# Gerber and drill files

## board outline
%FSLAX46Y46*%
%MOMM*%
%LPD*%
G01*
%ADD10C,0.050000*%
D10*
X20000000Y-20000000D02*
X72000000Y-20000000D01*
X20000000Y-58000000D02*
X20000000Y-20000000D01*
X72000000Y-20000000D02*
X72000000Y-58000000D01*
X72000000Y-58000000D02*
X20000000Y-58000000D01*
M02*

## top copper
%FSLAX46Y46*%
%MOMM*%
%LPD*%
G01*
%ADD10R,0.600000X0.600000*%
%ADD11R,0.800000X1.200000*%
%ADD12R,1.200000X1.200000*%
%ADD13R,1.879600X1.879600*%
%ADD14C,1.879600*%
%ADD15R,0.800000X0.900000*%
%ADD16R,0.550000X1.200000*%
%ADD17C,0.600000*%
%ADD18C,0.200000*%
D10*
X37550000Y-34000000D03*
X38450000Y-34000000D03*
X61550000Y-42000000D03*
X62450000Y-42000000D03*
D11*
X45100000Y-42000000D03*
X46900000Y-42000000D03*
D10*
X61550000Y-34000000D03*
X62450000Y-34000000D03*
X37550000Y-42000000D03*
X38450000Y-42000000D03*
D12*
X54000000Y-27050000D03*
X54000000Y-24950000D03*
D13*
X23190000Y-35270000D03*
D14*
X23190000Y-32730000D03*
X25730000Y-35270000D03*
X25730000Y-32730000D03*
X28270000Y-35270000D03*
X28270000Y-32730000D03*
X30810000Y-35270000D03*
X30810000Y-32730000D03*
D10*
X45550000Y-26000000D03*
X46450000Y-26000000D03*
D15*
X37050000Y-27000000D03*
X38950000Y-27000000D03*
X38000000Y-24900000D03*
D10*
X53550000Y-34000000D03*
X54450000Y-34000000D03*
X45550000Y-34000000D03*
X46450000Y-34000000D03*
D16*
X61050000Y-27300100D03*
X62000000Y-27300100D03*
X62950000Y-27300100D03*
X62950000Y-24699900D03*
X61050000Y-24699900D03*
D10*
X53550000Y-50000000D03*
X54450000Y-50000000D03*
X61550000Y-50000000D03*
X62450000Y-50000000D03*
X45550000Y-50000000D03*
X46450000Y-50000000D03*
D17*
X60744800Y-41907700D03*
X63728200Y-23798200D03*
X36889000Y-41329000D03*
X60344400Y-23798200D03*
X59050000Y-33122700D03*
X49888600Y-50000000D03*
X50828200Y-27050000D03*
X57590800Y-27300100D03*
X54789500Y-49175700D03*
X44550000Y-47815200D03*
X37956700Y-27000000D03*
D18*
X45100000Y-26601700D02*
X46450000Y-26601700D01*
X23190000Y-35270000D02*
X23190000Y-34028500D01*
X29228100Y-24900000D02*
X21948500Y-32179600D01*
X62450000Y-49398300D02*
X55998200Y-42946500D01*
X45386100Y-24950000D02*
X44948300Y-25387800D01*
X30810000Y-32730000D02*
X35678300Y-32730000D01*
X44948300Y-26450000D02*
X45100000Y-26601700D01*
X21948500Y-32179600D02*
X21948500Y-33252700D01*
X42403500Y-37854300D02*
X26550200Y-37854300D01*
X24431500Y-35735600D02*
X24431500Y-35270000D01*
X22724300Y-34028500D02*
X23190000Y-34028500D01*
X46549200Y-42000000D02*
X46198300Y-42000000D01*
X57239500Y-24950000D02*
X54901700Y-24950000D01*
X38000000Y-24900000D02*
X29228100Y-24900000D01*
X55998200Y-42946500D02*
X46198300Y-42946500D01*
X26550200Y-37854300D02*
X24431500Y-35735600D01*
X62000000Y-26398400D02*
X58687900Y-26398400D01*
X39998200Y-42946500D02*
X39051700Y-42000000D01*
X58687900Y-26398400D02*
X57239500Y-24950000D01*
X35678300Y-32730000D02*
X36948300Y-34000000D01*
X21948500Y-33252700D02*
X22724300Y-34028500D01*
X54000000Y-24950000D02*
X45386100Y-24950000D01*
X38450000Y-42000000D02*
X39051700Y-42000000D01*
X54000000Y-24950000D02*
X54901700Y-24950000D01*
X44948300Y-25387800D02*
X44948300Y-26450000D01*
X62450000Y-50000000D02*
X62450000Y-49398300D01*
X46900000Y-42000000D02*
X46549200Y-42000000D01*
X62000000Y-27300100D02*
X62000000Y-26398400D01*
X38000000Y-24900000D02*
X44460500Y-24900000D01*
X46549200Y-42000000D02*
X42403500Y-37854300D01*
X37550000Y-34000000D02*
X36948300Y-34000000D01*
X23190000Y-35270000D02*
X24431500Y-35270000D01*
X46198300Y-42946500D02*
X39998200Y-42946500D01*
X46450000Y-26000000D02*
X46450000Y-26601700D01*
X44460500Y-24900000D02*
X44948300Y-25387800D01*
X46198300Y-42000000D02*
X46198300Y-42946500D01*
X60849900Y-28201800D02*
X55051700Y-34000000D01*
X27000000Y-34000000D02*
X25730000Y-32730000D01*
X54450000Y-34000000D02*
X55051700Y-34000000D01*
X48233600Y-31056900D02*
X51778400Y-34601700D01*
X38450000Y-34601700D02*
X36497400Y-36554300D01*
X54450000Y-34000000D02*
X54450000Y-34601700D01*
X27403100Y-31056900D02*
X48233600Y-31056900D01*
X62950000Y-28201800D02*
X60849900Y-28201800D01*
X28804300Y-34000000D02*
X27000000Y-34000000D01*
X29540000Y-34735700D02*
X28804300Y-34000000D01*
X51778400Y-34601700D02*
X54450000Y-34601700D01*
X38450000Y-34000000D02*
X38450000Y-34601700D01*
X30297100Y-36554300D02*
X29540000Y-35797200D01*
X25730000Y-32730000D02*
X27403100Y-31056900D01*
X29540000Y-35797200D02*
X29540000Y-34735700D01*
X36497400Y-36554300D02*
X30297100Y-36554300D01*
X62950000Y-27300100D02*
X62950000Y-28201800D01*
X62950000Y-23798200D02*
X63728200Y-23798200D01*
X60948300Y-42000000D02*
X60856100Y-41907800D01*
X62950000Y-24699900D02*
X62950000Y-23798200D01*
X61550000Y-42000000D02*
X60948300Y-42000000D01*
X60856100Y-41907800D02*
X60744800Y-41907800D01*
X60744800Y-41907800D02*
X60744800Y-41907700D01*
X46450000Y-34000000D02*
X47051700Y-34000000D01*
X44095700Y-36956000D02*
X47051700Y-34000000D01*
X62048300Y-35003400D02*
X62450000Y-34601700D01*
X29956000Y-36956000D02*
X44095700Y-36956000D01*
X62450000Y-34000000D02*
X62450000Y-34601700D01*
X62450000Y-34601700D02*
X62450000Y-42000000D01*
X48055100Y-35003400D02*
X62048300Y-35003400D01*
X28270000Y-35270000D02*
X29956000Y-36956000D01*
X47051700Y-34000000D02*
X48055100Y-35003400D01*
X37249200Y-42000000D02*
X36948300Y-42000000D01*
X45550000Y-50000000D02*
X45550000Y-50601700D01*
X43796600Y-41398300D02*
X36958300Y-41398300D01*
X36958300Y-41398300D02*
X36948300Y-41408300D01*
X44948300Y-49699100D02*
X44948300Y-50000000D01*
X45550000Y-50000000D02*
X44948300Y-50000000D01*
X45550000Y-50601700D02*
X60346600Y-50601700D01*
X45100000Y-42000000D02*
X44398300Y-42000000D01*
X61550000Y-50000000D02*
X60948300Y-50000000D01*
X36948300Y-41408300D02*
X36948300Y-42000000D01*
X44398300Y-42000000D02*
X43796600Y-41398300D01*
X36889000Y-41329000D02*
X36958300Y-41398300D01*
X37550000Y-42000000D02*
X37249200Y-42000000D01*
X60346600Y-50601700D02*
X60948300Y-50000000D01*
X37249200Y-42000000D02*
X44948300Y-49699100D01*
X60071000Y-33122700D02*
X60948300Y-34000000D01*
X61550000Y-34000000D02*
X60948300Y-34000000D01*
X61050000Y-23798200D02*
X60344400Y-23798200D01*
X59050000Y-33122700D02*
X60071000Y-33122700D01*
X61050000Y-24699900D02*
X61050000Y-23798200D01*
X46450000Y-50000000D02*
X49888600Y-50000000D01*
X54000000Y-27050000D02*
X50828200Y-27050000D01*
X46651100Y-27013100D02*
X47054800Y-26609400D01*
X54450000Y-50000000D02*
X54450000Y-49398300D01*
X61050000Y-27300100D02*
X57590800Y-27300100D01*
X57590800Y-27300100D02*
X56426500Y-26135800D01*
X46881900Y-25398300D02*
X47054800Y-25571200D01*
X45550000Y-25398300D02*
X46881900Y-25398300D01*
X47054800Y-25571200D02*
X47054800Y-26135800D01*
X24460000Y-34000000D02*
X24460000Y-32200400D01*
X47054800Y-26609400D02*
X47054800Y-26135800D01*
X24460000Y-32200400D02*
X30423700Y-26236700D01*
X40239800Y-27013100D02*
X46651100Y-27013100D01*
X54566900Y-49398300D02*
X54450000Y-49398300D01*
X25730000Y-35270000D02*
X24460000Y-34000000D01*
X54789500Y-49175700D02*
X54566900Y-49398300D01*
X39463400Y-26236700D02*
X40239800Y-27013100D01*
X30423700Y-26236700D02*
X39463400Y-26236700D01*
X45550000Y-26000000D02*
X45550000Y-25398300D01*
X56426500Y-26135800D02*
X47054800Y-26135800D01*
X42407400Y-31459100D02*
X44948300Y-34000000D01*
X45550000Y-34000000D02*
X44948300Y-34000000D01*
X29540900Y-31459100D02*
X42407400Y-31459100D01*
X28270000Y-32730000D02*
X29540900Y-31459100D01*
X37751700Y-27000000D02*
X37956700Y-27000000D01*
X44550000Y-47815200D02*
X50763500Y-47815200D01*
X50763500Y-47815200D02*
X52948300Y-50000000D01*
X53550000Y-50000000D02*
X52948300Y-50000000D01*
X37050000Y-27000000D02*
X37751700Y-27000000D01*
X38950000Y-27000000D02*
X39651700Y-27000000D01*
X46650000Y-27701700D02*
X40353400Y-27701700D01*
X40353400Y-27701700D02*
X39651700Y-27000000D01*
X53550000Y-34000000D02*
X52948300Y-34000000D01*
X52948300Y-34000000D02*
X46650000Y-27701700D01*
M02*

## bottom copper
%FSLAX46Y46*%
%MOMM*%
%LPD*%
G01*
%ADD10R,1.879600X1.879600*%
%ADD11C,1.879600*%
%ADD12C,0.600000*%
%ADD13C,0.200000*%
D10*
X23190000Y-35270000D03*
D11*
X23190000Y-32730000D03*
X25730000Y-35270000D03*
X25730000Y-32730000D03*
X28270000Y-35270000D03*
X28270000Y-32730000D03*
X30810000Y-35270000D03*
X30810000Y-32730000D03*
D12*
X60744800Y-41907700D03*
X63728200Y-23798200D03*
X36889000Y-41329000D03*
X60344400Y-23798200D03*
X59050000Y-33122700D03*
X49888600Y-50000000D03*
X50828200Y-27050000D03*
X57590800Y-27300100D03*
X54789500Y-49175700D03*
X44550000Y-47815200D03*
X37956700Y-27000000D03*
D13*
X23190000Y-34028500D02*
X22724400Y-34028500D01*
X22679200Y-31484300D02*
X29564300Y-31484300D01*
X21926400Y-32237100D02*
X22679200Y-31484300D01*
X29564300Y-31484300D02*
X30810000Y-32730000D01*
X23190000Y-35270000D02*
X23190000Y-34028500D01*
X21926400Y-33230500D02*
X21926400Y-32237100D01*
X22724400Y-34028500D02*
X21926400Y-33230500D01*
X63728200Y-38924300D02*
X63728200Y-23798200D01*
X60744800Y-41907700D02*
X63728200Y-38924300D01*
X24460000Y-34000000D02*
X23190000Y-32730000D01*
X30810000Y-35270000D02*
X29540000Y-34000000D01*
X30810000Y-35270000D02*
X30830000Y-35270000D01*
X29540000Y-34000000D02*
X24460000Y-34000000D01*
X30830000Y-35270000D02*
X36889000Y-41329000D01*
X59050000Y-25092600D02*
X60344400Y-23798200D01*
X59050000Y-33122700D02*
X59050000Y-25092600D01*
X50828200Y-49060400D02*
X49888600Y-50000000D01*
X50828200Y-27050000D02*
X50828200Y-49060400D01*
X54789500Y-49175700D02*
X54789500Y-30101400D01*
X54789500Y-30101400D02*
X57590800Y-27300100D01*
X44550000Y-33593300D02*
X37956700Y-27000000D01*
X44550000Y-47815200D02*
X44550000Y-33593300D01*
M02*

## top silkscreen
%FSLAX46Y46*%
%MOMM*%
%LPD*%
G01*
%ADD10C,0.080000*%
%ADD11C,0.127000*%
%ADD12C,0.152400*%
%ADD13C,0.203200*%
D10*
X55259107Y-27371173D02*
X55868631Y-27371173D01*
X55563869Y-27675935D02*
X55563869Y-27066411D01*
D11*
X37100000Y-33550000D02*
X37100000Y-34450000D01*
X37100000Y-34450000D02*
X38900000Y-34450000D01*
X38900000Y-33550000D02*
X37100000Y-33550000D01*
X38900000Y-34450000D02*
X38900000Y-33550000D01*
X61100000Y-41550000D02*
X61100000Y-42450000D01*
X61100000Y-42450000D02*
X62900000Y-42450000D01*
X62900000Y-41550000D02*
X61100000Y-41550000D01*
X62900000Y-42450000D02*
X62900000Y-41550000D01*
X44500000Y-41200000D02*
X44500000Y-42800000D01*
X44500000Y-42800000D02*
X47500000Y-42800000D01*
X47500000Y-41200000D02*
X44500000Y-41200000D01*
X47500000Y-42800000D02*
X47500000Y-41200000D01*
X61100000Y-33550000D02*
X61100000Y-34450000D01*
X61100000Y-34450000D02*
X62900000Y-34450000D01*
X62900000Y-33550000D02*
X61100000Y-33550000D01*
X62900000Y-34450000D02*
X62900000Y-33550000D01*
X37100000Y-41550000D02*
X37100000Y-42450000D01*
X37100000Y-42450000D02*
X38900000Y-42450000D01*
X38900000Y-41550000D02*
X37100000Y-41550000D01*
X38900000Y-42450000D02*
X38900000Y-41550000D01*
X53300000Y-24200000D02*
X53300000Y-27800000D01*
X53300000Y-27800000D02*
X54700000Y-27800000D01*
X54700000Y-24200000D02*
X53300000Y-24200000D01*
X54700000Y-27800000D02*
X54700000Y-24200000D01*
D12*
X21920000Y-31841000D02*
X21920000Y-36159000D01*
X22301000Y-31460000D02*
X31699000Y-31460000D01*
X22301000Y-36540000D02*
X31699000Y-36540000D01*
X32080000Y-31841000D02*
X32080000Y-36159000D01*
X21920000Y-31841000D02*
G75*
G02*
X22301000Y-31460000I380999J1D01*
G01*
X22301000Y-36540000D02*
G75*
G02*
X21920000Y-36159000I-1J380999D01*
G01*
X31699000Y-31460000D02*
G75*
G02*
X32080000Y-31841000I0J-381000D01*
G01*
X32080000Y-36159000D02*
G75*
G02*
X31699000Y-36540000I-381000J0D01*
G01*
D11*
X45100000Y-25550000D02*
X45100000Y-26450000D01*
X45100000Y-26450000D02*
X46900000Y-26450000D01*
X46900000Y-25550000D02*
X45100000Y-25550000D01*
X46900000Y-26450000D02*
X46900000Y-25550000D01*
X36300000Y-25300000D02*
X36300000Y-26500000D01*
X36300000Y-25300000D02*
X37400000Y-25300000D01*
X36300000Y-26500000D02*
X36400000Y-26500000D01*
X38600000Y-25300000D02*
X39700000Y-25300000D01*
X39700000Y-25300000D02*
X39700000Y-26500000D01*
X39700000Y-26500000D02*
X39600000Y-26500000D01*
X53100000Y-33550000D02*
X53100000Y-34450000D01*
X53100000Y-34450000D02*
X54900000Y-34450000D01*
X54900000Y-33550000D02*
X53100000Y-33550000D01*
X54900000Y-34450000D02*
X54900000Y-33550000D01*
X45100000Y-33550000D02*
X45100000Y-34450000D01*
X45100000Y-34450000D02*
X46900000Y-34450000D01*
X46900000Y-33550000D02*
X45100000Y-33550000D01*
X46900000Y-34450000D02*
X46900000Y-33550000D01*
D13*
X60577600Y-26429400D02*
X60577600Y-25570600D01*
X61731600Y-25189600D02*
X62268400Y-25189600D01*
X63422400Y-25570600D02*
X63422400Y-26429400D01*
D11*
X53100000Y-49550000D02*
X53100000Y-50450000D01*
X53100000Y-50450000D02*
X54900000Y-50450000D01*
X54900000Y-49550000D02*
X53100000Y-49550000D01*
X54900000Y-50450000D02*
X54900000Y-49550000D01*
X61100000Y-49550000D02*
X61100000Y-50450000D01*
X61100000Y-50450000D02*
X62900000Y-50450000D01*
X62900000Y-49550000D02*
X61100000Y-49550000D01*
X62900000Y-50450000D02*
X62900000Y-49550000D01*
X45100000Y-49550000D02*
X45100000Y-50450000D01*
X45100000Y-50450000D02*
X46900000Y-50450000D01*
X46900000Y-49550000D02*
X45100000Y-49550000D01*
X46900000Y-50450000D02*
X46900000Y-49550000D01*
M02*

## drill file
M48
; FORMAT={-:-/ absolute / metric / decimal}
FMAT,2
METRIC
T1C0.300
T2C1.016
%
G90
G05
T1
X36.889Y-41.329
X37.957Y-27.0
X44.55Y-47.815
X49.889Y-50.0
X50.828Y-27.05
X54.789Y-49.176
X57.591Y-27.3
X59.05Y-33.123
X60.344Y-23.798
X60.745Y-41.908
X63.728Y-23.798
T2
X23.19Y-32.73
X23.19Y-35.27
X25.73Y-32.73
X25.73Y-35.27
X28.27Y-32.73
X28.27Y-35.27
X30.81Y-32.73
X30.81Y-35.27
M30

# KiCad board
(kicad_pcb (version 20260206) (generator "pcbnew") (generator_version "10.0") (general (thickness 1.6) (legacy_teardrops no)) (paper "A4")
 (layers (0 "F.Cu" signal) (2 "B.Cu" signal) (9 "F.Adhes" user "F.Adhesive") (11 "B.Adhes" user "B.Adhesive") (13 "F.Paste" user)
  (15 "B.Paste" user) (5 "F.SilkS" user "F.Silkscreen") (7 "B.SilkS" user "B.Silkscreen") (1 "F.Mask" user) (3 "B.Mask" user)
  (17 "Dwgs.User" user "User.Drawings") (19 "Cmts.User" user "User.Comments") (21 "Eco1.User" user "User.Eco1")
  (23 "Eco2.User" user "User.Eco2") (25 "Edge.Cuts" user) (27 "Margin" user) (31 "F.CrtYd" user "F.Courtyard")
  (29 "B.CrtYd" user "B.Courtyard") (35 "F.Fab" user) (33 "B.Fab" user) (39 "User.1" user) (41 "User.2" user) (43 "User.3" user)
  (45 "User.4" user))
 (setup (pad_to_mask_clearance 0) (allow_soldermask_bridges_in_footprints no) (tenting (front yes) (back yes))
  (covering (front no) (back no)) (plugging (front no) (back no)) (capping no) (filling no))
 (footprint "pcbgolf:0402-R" (layer "F.Cu") (at 38 34)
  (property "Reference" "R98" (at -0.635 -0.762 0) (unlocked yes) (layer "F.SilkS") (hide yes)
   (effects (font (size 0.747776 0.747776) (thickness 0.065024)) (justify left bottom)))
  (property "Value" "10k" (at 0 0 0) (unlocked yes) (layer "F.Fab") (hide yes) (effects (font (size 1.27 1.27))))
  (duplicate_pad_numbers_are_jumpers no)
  (fp_line (start -0.9 -0.45) (end -0.9 0.45) (stroke (width 0.127) (type solid)) (layer "F.SilkS"))
  (fp_line (start -0.9 0.45) (end 0.9 0.45) (stroke (width 0.127) (type solid)) (layer "F.SilkS"))
  (fp_line (start 0.9 -0.45) (end -0.9 -0.45) (stroke (width 0.127) (type solid)) (layer "F.SilkS"))
  (fp_line (start 0.9 0.45) (end 0.9 -0.45) (stroke (width 0.127) (type solid)) (layer "F.SilkS"))
  (pad "1" smd rect (at -0.45 0) (size 0.6 0.6) (layers "F.Cu" "F.Mask" "F.Paste") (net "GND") (solder_mask_margin 0.0508)
   (solder_paste_margin 0) (thermal_bridge_angle 0))
  (pad "2" smd rect (at 0.45 0) (size 0.6 0.6) (layers "F.Cu" "F.Mask" "F.Paste") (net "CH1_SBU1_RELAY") (solder_mask_margin 0.0508)
   (solder_paste_margin 0) (thermal_bridge_angle 0)))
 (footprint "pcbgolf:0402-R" (layer "F.Cu") (at 62 42)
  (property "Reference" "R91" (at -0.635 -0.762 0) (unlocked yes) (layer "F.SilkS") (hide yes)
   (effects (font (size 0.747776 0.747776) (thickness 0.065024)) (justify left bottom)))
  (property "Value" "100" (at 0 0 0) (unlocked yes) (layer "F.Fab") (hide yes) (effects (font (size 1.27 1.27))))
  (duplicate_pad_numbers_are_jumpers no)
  (fp_line (start -0.9 -0.45) (end -0.9 0.45) (stroke (width 0.127) (type solid)) (layer "F.SilkS"))
  (fp_line (start -0.9 0.45) (end 0.9 0.45) (stroke (width 0.127) (type solid)) (layer "F.SilkS"))
  (fp_line (start 0.9 -0.45) (end -0.9 -0.45) (stroke (width 0.127) (type solid)) (layer "F.SilkS"))
  (fp_line (start 0.9 0.45) (end 0.9 -0.45) (stroke (width 0.127) (type solid)) (layer "F.SilkS"))
  (pad "1" smd rect (at -0.45 0) (size 0.6 0.6) (layers "F.Cu" "F.Mask" "F.Paste") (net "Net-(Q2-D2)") (solder_mask_margin 0.0508)
   (solder_paste_margin 0) (thermal_bridge_angle 0))
  (pad "2" smd rect (at 0.45 0) (size 0.6 0.6) (layers "F.Cu" "F.Mask" "F.Paste") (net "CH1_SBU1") (solder_mask_margin 0.0508)
   (solder_paste_margin 0) (thermal_bridge_angle 0)))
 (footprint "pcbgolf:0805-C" (layer "F.Cu") (at 46 42)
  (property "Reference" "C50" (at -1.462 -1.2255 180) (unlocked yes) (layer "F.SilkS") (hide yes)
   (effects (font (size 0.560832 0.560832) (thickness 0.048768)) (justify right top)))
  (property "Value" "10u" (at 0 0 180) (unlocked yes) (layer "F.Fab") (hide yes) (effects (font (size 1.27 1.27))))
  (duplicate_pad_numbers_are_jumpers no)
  (fp_line (start -1.5 -0.8) (end -1.5 0.8) (stroke (width 0.127) (type solid)) (layer "F.SilkS"))
  (fp_line (start -1.5 0.8) (end 1.5 0.8) (stroke (width 0.127) (type solid)) (layer "F.SilkS"))
  (fp_line (start 1.5 -0.8) (end -1.5 -0.8) (stroke (width 0.127) (type solid)) (layer "F.SilkS"))
  (fp_line (start 1.5 0.8) (end 1.5 -0.8) (stroke (width 0.127) (type solid)) (layer "F.SilkS"))
  (pad "1" smd rect (at -0.9 0) (size 0.8 1.2) (layers "F.Cu" "F.Mask" "F.Paste") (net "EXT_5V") (solder_mask_margin 0.0508)
   (solder_paste_margin 0) (thermal_bridge_angle 0))
  (pad "2" smd rect (at 0.9 0) (size 0.8 1.2) (layers "F.Cu" "F.Mask" "F.Paste") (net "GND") (solder_mask_margin 0.0508)
   (solder_paste_margin 0) (thermal_bridge_angle 0)))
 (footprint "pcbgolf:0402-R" (layer "F.Cu") (at 62 34)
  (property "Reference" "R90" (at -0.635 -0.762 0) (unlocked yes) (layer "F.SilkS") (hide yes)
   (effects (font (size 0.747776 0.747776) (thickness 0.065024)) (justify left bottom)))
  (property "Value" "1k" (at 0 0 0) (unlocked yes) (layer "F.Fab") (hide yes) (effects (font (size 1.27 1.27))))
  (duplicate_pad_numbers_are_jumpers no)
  (fp_line (start -0.9 -0.45) (end -0.9 0.45) (stroke (width 0.127) (type solid)) (layer "F.SilkS"))
  (fp_line (start -0.9 0.45) (end 0.9 0.45) (stroke (width 0.127) (type solid)) (layer "F.SilkS"))
  (fp_line (start 0.9 -0.45) (end -0.9 -0.45) (stroke (width 0.127) (type solid)) (layer "F.SilkS"))
  (fp_line (start 0.9 0.45) (end 0.9 -0.45) (stroke (width 0.127) (type solid)) (layer "F.SilkS"))
  (pad "1" smd rect (at -0.45 0) (size 0.6 0.6) (layers "F.Cu" "F.Mask" "F.Paste") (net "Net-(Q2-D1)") (solder_mask_margin 0.0508)
   (solder_paste_margin 0) (thermal_bridge_angle 0))
  (pad "2" smd rect (at 0.45 0) (size 0.6 0.6) (layers "F.Cu" "F.Mask" "F.Paste") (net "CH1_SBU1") (solder_mask_margin 0.0508)
   (solder_paste_margin 0) (thermal_bridge_angle 0)))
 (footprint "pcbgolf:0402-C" (layer "F.Cu") (at 38 42)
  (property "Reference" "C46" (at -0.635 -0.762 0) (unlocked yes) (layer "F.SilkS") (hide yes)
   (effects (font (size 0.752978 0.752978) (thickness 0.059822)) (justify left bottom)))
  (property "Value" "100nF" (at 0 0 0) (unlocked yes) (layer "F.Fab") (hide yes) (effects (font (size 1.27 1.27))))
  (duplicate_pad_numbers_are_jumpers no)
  (fp_line (start -0.9 -0.45) (end -0.9 0.45) (stroke (width 0.127) (type solid)) (layer "F.SilkS"))
  (fp_line (start -0.9 0.45) (end 0.9 0.45) (stroke (width 0.127) (type solid)) (layer "F.SilkS"))
  (fp_line (start 0.9 -0.45) (end -0.9 -0.45) (stroke (width 0.127) (type solid)) (layer "F.SilkS"))
  (fp_line (start 0.9 0.45) (end 0.9 -0.45) (stroke (width 0.127) (type solid)) (layer "F.SilkS"))
  (pad "1" smd rect (at -0.45 0) (size 0.6 0.6) (layers "F.Cu" "F.Mask" "F.Paste") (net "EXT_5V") (solder_mask_margin 0.0508)
   (solder_paste_margin 0) (thermal_bridge_angle 0))
  (pad "2" smd rect (at 0.45 0) (size 0.6 0.6) (layers "F.Cu" "F.Mask" "F.Paste") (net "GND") (solder_mask_margin 0.0508)
   (solder_paste_margin 0) (thermal_bridge_angle 0)))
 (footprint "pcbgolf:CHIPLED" (layer "F.Cu") (at 54 26)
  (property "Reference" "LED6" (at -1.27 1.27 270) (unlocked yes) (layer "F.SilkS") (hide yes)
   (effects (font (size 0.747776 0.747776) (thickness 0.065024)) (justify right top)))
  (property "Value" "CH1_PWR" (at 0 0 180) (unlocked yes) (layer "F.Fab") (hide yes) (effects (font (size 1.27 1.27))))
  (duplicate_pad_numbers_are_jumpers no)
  (fp_line (start -0.7 -1.8) (end -0.7 1.8) (stroke (width 0.127) (type solid)) (layer "F.SilkS"))
  (fp_line (start -0.7 1.8) (end 0.7 1.8) (stroke (width 0.127) (type solid)) (layer "F.SilkS"))
  (fp_line (start 0.7 -1.8) (end -0.7 -1.8) (stroke (width 0.127) (type solid)) (layer "F.SilkS"))
  (fp_line (start 0.7 1.8) (end 0.7 -1.8) (stroke (width 0.127) (type solid)) (layer "F.SilkS"))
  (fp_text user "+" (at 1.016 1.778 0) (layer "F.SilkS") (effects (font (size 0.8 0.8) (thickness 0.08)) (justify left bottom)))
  (pad "A" smd rect (at 0 1.05) (size 1.2 1.2) (layers "F.Cu" "F.Mask" "F.Paste") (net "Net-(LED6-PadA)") (solder_mask_margin 0.0508)
   (solder_paste_margin 0) (thermal_bridge_angle 0))
  (pad "C" smd rect (at 0 -1.05) (size 1.2 1.2) (layers "F.Cu" "F.Mask" "F.Paste") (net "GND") (solder_mask_margin 0.0508)
   (solder_paste_margin 0) (thermal_bridge_angle 0)))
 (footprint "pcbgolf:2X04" (layer "F.Cu") (at 27 34)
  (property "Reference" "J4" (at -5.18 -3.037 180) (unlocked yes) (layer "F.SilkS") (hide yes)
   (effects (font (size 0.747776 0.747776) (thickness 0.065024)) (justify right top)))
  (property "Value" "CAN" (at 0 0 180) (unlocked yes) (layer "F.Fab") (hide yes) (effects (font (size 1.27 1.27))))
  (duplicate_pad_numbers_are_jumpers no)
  (fp_line (start -5.08 -2.159) (end -5.08 2.159) (stroke (width 0.1524) (type solid)) (layer "F.SilkS"))
  (fp_line (start -4.699 -2.54) (end 4.699 -2.54) (stroke (width 0.1524) (type solid)) (layer "F.SilkS"))
  (fp_line (start -4.699 2.54) (end 4.699 2.54) (stroke (width 0.1524) (type solid)) (layer "F.SilkS"))
  (fp_line (start 5.08 -2.159) (end 5.08 2.159) (stroke (width 0.1524) (type solid)) (layer "F.SilkS"))
  (fp_arc (start -5.08 -2.159) (mid -4.968408 -2.428408) (end -4.699 -2.54) (stroke (width 0.1524) (type solid)) (layer "F.SilkS"))
  (fp_arc (start -4.699 2.54) (mid -4.968408 2.428408) (end -5.08 2.159) (stroke (width 0.1524) (type solid)) (layer "F.SilkS"))
  (fp_arc (start 4.699 -2.54) (mid 4.968408 -2.428408) (end 5.08 -2.159) (stroke (width 0.1524) (type solid)) (layer "F.SilkS"))
  (fp_arc (start 5.08 2.159) (mid 4.968408 2.428408) (end 4.699 2.54) (stroke (width 0.1524) (type solid)) (layer "F.SilkS"))
  (pad "1" thru_hole rect (at -3.81 1.27 90) (size 1.8796 1.8796) (drill 1.016) (layers "*.Cu" "*.Mask") (remove_unused_layers no)
   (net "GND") (solder_mask_margin 0.0508) (thermal_bridge_angle 0))
  (pad "2" thru_hole circle (at -3.81 -1.27 90) (size 1.8796 1.8796) (drill 1.016) (layers "*.Cu" "*.Mask") (remove_unused_layers no)
   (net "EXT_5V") (solder_mask_margin 0.0508) (thermal_bridge_angle 0))
  (pad "3" thru_hole circle (at -1.27 1.27 90) (size 1.8796 1.8796) (drill 1.016) (layers "*.Cu" "*.Mask") (remove_unused_layers no)
   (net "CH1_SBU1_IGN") (solder_mask_margin 0.0508) (thermal_bridge_angle 0))
  (pad "4" thru_hole circle (at -1.27 -1.27 90) (size 1.8796 1.8796) (drill 1.016) (layers "*.Cu" "*.Mask") (remove_unused_layers no)
   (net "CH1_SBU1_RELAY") (solder_mask_margin 0.0508) (thermal_bridge_angle 0))
  (pad "5" thru_hole circle (at 1.27 1.27 90) (size 1.8796 1.8796) (drill 1.016) (layers "*.Cu" "*.Mask") (remove_unused_layers no)
   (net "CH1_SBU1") (solder_mask_margin 0.0508) (thermal_bridge_angle 0))
  (pad "6" thru_hole circle (at 1.27 -1.27 90) (size 1.8796 1.8796) (drill 1.016) (layers "*.Cu" "*.Mask") (remove_unused_layers no)
   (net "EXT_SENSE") (solder_mask_margin 0.0508) (thermal_bridge_angle 0))
  (pad "7" thru_hole circle (at 3.81 1.27 90) (size 1.8796 1.8796) (drill 1.016) (layers "*.Cu" "*.Mask") (remove_unused_layers no)
   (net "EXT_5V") (solder_mask_margin 0.0508) (thermal_bridge_angle 0))
  (pad "8" thru_hole circle (at 3.81 -1.27 90) (size 1.8796 1.8796) (drill 1.016) (layers "*.Cu" "*.Mask") (remove_unused_layers no)
   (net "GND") (solder_mask_margin 0.0508) (thermal_bridge_angle 0)))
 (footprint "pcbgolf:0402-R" (layer "F.Cu") (at 46 26)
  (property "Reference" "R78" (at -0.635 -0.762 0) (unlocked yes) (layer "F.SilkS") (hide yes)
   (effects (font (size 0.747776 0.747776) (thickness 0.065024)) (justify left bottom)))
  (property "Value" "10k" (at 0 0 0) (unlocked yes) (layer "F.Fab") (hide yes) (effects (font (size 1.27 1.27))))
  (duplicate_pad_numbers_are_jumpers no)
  (fp_line (start -0.9 -0.45) (end -0.9 0.45) (stroke (width 0.127) (type solid)) (layer "F.SilkS"))
  (fp_line (start -0.9 0.45) (end 0.9 0.45) (stroke (width 0.127) (type solid)) (layer "F.SilkS"))
  (fp_line (start 0.9 -0.45) (end -0.9 -0.45) (stroke (width 0.127) (type solid)) (layer "F.SilkS"))
  (fp_line (start 0.9 0.45) (end 0.9 -0.45) (stroke (width 0.127) (type solid)) (layer "F.SilkS"))
  (pad "1" smd rect (at -0.45 0) (size 0.6 0.6) (layers "F.Cu" "F.Mask" "F.Paste") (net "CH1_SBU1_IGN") (solder_mask_margin 0.0508)
   (solder_paste_margin 0) (thermal_bridge_angle 0))
  (pad "2" smd rect (at 0.45 0) (size 0.6 0.6) (layers "F.Cu" "F.Mask" "F.Paste") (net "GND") (solder_mask_margin 0.0508)
   (solder_paste_margin 0) (thermal_bridge_angle 0)))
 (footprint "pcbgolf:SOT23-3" (layer "F.Cu") (at 38 26)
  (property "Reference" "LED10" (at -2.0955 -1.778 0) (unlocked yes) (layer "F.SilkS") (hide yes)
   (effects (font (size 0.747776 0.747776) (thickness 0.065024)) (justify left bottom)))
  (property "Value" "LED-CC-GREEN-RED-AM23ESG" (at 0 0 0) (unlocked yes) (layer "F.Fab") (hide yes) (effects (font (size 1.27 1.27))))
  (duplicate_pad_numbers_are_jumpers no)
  (fp_line (start -1.7 -0.7) (end -1.7 0.5) (stroke (width 0.127) (type solid)) (layer "F.SilkS"))
  (fp_line (start -1.7 -0.7) (end -0.6 -0.7) (stroke (width 0.127) (type solid)) (layer "F.SilkS"))
  (fp_line (start -1.7 0.5) (end -1.6 0.5) (stroke (width 0.127) (type solid)) (layer "F.SilkS"))
  (fp_line (start 0.6 -0.7) (end 1.7 -0.7) (stroke (width 0.127) (type solid)) (layer "F.SilkS"))
  (fp_line (start 1.7 -0.7) (end 1.7 0.5) (stroke (width 0.127) (type solid)) (layer "F.SilkS"))
  (fp_line (start 1.7 0.5) (end 1.6 0.5) (stroke (width 0.127) (type solid)) (layer "F.SilkS"))
  (pad "1" smd rect (at -0.95 1) (size 0.8 0.9) (layers "F.Cu" "F.Mask" "F.Paste") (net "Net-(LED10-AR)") (solder_mask_margin 0.0508)
   (solder_paste_margin 0) (thermal_bridge_angle 0))
  (pad "2" smd rect (at 0.95 1) (size 0.8 0.9) (layers "F.Cu" "F.Mask" "F.Paste") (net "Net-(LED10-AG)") (solder_mask_margin 0.0508)
   (solder_paste_margin 0) (thermal_bridge_angle 0))
  (pad "3" smd rect (at 0 -1.1) (size 0.8 0.9) (layers "F.Cu" "F.Mask" "F.Paste") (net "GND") (solder_mask_margin 0.0508)
   (solder_paste_margin 0) (thermal_bridge_angle 0)))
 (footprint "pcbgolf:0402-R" (layer "F.Cu") (at 54 34)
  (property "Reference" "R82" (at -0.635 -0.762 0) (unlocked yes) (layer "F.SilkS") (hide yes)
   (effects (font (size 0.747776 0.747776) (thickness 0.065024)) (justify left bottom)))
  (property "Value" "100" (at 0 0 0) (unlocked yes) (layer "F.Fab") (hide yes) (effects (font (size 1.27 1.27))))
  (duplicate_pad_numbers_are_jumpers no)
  (fp_line (start -0.9 -0.45) (end -0.9 0.45) (stroke (width 0.127) (type solid)) (layer "F.SilkS"))
  (fp_line (start -0.9 0.45) (end 0.9 0.45) (stroke (width 0.127) (type solid)) (layer "F.SilkS"))
  (fp_line (start 0.9 -0.45) (end -0.9 -0.45) (stroke (width 0.127) (type solid)) (layer "F.SilkS"))
  (fp_line (start 0.9 0.45) (end 0.9 -0.45) (stroke (width 0.127) (type solid)) (layer "F.SilkS"))
  (pad "1" smd rect (at -0.45 0) (size 0.6 0.6) (layers "F.Cu" "F.Mask" "F.Paste") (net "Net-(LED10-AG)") (solder_mask_margin 0.0508)
   (solder_paste_margin 0) (thermal_bridge_angle 0))
  (pad "2" smd rect (at 0.45 0) (size 0.6 0.6) (layers "F.Cu" "F.Mask" "F.Paste") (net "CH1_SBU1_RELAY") (solder_mask_margin 0.0508)
   (solder_paste_margin 0) (thermal_bridge_angle 0)))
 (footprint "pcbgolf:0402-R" (layer "F.Cu") (at 46 34)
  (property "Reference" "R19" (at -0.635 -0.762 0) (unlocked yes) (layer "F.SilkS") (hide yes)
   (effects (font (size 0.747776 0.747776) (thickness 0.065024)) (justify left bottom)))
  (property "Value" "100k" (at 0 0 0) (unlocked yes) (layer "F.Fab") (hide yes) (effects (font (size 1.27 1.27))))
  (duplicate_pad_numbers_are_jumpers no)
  (fp_line (start -0.9 -0.45) (end -0.9 0.45) (stroke (width 0.127) (type solid)) (layer "F.SilkS"))
  (fp_line (start -0.9 0.45) (end 0.9 0.45) (stroke (width 0.127) (type solid)) (layer "F.SilkS"))
  (fp_line (start 0.9 -0.45) (end -0.9 -0.45) (stroke (width 0.127) (type solid)) (layer "F.SilkS"))
  (fp_line (start 0.9 0.45) (end 0.9 -0.45) (stroke (width 0.127) (type solid)) (layer "F.SilkS"))
  (pad "1" smd rect (at -0.45 0) (size 0.6 0.6) (layers "F.Cu" "F.Mask" "F.Paste") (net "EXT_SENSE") (solder_mask_margin 0.0508)
   (solder_paste_margin 0) (thermal_bridge_angle 0))
  (pad "2" smd rect (at 0.45 0) (size 0.6 0.6) (layers "F.Cu" "F.Mask" "F.Paste") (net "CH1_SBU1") (solder_mask_margin 0.0508)
   (solder_paste_margin 0) (thermal_bridge_angle 0)))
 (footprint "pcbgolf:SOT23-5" (layer "F.Cu") (at 62 26)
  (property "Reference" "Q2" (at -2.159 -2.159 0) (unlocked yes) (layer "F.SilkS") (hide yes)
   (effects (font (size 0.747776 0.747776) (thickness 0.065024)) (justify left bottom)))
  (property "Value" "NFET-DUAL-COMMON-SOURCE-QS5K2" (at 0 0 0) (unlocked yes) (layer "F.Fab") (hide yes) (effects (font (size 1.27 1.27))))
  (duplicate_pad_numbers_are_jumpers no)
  (fp_line (start -1.4224 0.4294) (end -1.4224 -0.4294) (stroke (width 0.2032) (type solid)) (layer "F.SilkS"))
  (fp_line (start -0.2684 -0.8104) (end 0.2684 -0.8104) (stroke (width 0.2032) (type solid)) (layer "F.SilkS"))
  (fp_line (start 1.4224 -0.4294) (end 1.4224 0.4294) (stroke (width 0.2032) (type solid)) (layer "F.SilkS"))
  (pad "1" smd rect (at -0.95 1.3001) (size 0.55 1.2) (layers "F.Cu" "F.Mask" "F.Paste") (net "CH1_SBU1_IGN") (solder_mask_margin 0.0508)
   (solder_paste_margin 0) (thermal_bridge_angle 0))
  (pad "2" smd rect (at 0 1.3001) (size 0.55 1.2) (layers "F.Cu" "F.Mask" "F.Paste") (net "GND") (solder_mask_margin 0.0508)
   (solder_paste_margin 0) (thermal_bridge_angle 0))
  (pad "3" smd rect (at 0.95 1.3001) (size 0.55 1.2) (layers "F.Cu" "F.Mask" "F.Paste") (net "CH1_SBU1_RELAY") (solder_mask_margin 0.0508)
   (solder_paste_margin 0) (thermal_bridge_angle 0))
  (pad "4" smd rect (at 0.95 -1.3001) (size 0.55 1.2) (layers "F.Cu" "F.Mask" "F.Paste") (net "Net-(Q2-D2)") (solder_mask_margin 0.0508)
   (solder_paste_margin 0) (thermal_bridge_angle 0))
  (pad "5" smd rect (at -0.95 -1.3001) (size 0.55 1.2) (layers "F.Cu" "F.Mask" "F.Paste") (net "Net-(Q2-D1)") (solder_mask_margin 0.0508)
   (solder_paste_margin 0) (thermal_bridge_angle 0)))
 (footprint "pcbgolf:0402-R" (layer "F.Cu") (at 54 50)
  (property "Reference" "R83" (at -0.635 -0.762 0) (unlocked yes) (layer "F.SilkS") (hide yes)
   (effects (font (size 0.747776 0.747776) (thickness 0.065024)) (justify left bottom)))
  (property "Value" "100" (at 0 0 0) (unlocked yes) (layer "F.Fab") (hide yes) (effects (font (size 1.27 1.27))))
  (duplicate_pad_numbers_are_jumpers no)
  (fp_line (start -0.9 -0.45) (end -0.9 0.45) (stroke (width 0.127) (type solid)) (layer "F.SilkS"))
  (fp_line (start -0.9 0.45) (end 0.9 0.45) (stroke (width 0.127) (type solid)) (layer "F.SilkS"))
  (fp_line (start 0.9 -0.45) (end -0.9 -0.45) (stroke (width 0.127) (type solid)) (layer "F.SilkS"))
  (fp_line (start 0.9 0.45) (end 0.9 -0.45) (stroke (width 0.127) (type solid)) (layer "F.SilkS"))
  (pad "1" smd rect (at -0.45 0) (size 0.6 0.6) (layers "F.Cu" "F.Mask" "F.Paste") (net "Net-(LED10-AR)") (solder_mask_margin 0.0508)
   (solder_paste_margin 0) (thermal_bridge_angle 0))
  (pad "2" smd rect (at 0.45 0) (size 0.6 0.6) (layers "F.Cu" "F.Mask" "F.Paste") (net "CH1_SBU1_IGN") (solder_mask_margin 0.0508)
   (solder_paste_margin 0) (thermal_bridge_angle 0)))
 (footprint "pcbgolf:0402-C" (layer "F.Cu") (at 62 50)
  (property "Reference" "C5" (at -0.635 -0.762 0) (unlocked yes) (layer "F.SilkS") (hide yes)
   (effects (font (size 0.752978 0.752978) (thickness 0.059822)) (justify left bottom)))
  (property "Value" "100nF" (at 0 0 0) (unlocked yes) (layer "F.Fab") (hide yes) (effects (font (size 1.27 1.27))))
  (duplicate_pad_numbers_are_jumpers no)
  (fp_line (start -0.9 -0.45) (end -0.9 0.45) (stroke (width 0.127) (type solid)) (layer "F.SilkS"))
  (fp_line (start -0.9 0.45) (end 0.9 0.45) (stroke (width 0.127) (type solid)) (layer "F.SilkS"))
  (fp_line (start 0.9 -0.45) (end -0.9 -0.45) (stroke (width 0.127) (type solid)) (layer "F.SilkS"))
  (fp_line (start 0.9 0.45) (end 0.9 -0.45) (stroke (width 0.127) (type solid)) (layer "F.SilkS"))
  (pad "1" smd rect (at -0.45 0) (size 0.6 0.6) (layers "F.Cu" "F.Mask" "F.Paste") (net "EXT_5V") (solder_mask_margin 0.0508)
   (solder_paste_margin 0) (thermal_bridge_angle 0))
  (pad "2" smd rect (at 0.45 0) (size 0.6 0.6) (layers "F.Cu" "F.Mask" "F.Paste") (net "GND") (solder_mask_margin 0.0508)
   (solder_paste_margin 0) (thermal_bridge_angle 0)))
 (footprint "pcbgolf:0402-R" (layer "F.Cu") (at 46 50)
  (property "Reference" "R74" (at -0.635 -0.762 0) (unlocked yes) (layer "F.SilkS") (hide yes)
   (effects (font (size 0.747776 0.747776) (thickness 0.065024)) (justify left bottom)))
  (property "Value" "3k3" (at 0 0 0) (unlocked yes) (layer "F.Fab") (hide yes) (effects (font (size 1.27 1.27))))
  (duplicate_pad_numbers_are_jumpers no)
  (fp_line (start -0.9 -0.45) (end -0.9 0.45) (stroke (width 0.127) (type solid)) (layer "F.SilkS"))
  (fp_line (start -0.9 0.45) (end 0.9 0.45) (stroke (width 0.127) (type solid)) (layer "F.SilkS"))
  (fp_line (start 0.9 -0.45) (end -0.9 -0.45) (stroke (width 0.127) (type solid)) (layer "F.SilkS"))
  (fp_line (start 0.9 0.45) (end 0.9 -0.45) (stroke (width 0.127) (type solid)) (layer "F.SilkS"))
  (pad "1" smd rect (at -0.45 0) (size 0.6 0.6) (layers "F.Cu" "F.Mask" "F.Paste") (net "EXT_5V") (solder_mask_margin 0.0508)
   (solder_paste_margin 0) (thermal_bridge_angle 0))
  (pad "2" smd rect (at 0.45 0) (size 0.6 0.6) (layers "F.Cu" "F.Mask" "F.Paste") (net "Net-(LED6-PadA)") (solder_mask_margin 0.0508)
   (solder_paste_margin 0) (thermal_bridge_angle 0)))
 (gr_line (start 20 20) (end 72 20) (stroke (width 0.05) (type default)) (layer "Edge.Cuts"))
 (gr_line (start 20 58) (end 20 20) (stroke (width 0.05) (type default)) (layer "Edge.Cuts"))
 (gr_line (start 72 20) (end 72 58) (stroke (width 0.05) (type default)) (layer "Edge.Cuts"))
 (gr_line (start 72 58) (end 20 58) (stroke (width 0.05) (type default)) (layer "Edge.Cuts"))
 (segment (start 45.1 26.6017) (end 46.45 26.6017) (width 0.2) (layer "F.Cu") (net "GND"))
 (segment (start 23.19 35.27) (end 23.19 34.0285) (width 0.2) (layer "F.Cu") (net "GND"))
 (segment (start 29.2281 24.9) (end 21.9485 32.1796) (width 0.2) (layer "F.Cu") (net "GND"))
 (segment (start 62.45 49.3983) (end 55.9982 42.9465) (width 0.2) (layer "F.Cu") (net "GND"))
 (segment (start 45.3861 24.95) (end 44.9483 25.3878) (width 0.2) (layer "F.Cu") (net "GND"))
 (segment (start 30.81 32.73) (end 35.6783 32.73) (width 0.2) (layer "F.Cu") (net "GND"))
 (segment (start 44.9483 26.45) (end 45.1 26.6017) (width 0.2) (layer "F.Cu") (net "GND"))
 (segment (start 21.9485 32.1796) (end 21.9485 33.2527) (width 0.2) (layer "F.Cu") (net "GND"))
 (segment (start 42.4035 37.8543) (end 26.5502 37.8543) (width 0.2) (layer "F.Cu") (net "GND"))
 (segment (start 24.4315 35.7356) (end 24.4315 35.27) (width 0.2) (layer "F.Cu") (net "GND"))
 (segment (start 22.7243 34.0285) (end 23.19 34.0285) (width 0.2) (layer "F.Cu") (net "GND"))
 (segment (start 46.5492 42) (end 46.1983 42) (width 0.2) (layer "F.Cu") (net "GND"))
 (segment (start 57.2395 24.95) (end 54.9017 24.95) (width 0.2) (layer "F.Cu") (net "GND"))
 (segment (start 38 24.9) (end 29.2281 24.9) (width 0.2) (layer "F.Cu") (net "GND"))
 (segment (start 55.9982 42.9465) (end 46.1983 42.9465) (width 0.2) (layer "F.Cu") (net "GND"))
 (segment (start 26.5502 37.8543) (end 24.4315 35.7356) (width 0.2) (layer "F.Cu") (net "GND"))
 (segment (start 62 26.3984) (end 58.6879 26.3984) (width 0.2) (layer "F.Cu") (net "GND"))
 (segment (start 39.9982 42.9465) (end 39.0517 42) (width 0.2) (layer "F.Cu") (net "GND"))
 (segment (start 58.6879 26.3984) (end 57.2395 24.95) (width 0.2) (layer "F.Cu") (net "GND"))
 (segment (start 35.6783 32.73) (end 36.9483 34) (width 0.2) (layer "F.Cu") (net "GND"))
 (segment (start 21.9485 33.2527) (end 22.7243 34.0285) (width 0.2) (layer "F.Cu") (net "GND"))
 (segment (start 54 24.95) (end 45.3861 24.95) (width 0.2) (layer "F.Cu") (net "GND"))
 (segment (start 38.45 42) (end 39.0517 42) (width 0.2) (layer "F.Cu") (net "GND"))
 (segment (start 54 24.95) (end 54.9017 24.95) (width 0.2) (layer "F.Cu") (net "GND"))
 (segment (start 44.9483 25.3878) (end 44.9483 26.45) (width 0.2) (layer "F.Cu") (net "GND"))
 (segment (start 62.45 50) (end 62.45 49.3983) (width 0.2) (layer "F.Cu") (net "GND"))
 (segment (start 46.9 42) (end 46.5492 42) (width 0.2) (layer "F.Cu") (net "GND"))
 (segment (start 62 27.3001) (end 62 26.3984) (width 0.2) (layer "F.Cu") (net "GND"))
 (segment (start 38 24.9) (end 44.4605 24.9) (width 0.2) (layer "F.Cu") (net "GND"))
 (segment (start 46.5492 42) (end 42.4035 37.8543) (width 0.2) (layer "F.Cu") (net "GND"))
 (segment (start 37.55 34) (end 36.9483 34) (width 0.2) (layer "F.Cu") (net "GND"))
 (segment (start 23.19 35.27) (end 24.4315 35.27) (width 0.2) (layer "F.Cu") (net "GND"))
 (segment (start 46.1983 42.9465) (end 39.9982 42.9465) (width 0.2) (layer "F.Cu") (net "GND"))
 (segment (start 46.45 26) (end 46.45 26.6017) (width 0.2) (layer "F.Cu") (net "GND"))
 (segment (start 44.4605 24.9) (end 44.9483 25.3878) (width 0.2) (layer "F.Cu") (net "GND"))
 (segment (start 46.1983 42) (end 46.1983 42.9465) (width 0.2) (layer "F.Cu") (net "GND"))
 (segment (start 23.19 34.0285) (end 22.7244 34.0285) (width 0.2) (layer "B.Cu") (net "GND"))
 (segment (start 22.6792 31.4843) (end 29.5643 31.4843) (width 0.2) (layer "B.Cu") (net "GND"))
 (segment (start 21.9264 32.2371) (end 22.6792 31.4843) (width 0.2) (layer "B.Cu") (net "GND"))
 (segment (start 29.5643 31.4843) (end 30.81 32.73) (width 0.2) (layer "B.Cu") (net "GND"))
 (segment (start 23.19 35.27) (end 23.19 34.0285) (width 0.2) (layer "B.Cu") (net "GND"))
 (segment (start 21.9264 33.2305) (end 21.9264 32.2371) (width 0.2) (layer "B.Cu") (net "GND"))
 (segment (start 22.7244 34.0285) (end 21.9264 33.2305) (width 0.2) (layer "B.Cu") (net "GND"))
 (segment (start 60.8499 28.2018) (end 55.0517 34) (width 0.2) (layer "F.Cu") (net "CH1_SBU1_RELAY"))
 (segment (start 27 34) (end 25.73 32.73) (width 0.2) (layer "F.Cu") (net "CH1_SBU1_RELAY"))
 (segment (start 54.45 34) (end 55.0517 34) (width 0.2) (layer "F.Cu") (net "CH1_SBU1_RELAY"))
 (segment (start 48.2336 31.0569) (end 51.7784 34.6017) (width 0.2) (layer "F.Cu") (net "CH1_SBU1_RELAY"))
 (segment (start 38.45 34.6017) (end 36.4974 36.5543) (width 0.2) (layer "F.Cu") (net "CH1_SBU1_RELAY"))
 (segment (start 54.45 34) (end 54.45 34.6017) (width 0.2) (layer "F.Cu") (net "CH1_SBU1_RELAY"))
 (segment (start 27.4031 31.0569) (end 48.2336 31.0569) (width 0.2) (layer "F.Cu") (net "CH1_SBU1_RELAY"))
 (segment (start 62.95 28.2018) (end 60.8499 28.2018) (width 0.2) (layer "F.Cu") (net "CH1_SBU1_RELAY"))
 (segment (start 28.8043 34) (end 27 34) (width 0.2) (layer "F.Cu") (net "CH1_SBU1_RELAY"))
 (segment (start 29.54 34.7357) (end 28.8043 34) (width 0.2) (layer "F.Cu") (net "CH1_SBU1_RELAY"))
 (segment (start 51.7784 34.6017) (end 54.45 34.6017) (width 0.2) (layer "F.Cu") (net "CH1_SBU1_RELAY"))
 (segment (start 38.45 34) (end 38.45 34.6017) (width 0.2) (layer "F.Cu") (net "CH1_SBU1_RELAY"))
 (segment (start 30.2971 36.5543) (end 29.54 35.7972) (width 0.2) (layer "F.Cu") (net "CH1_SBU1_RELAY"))
 (segment (start 25.73 32.73) (end 27.4031 31.0569) (width 0.2) (layer "F.Cu") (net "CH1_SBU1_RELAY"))
 (segment (start 29.54 35.7972) (end 29.54 34.7357) (width 0.2) (layer "F.Cu") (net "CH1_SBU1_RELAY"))
 (segment (start 36.4974 36.5543) (end 30.2971 36.5543) (width 0.2) (layer "F.Cu") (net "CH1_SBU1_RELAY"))
 (segment (start 62.95 27.3001) (end 62.95 28.2018) (width 0.2) (layer "F.Cu") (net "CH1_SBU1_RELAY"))
 (segment (start 62.95 23.7982) (end 63.7282 23.7982) (width 0.2) (layer "F.Cu") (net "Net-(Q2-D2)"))
 (segment (start 60.9483 42) (end 60.8561 41.9078) (width 0.2) (layer "F.Cu") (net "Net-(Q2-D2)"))
 (segment (start 62.95 24.6999) (end 62.95 23.7982) (width 0.2) (layer "F.Cu") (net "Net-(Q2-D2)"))
 (segment (start 61.55 42) (end 60.9483 42) (width 0.2) (layer "F.Cu") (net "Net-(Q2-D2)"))
 (segment (start 60.8561 41.9078) (end 60.7448 41.9078) (width 0.2) (layer "F.Cu") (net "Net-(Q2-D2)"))
 (segment (start 60.7448 41.9078) (end 60.7448 41.9077) (width 0.2) (layer "F.Cu") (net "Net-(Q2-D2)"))
 (via (at 60.7448 41.9077) (size 0.6) (drill 0.3) (layers "F.Cu" "B.Cu") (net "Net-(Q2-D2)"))
 (via (at 63.7282 23.7982) (size 0.6) (drill 0.3) (layers "F.Cu" "B.Cu") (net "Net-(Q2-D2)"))
 (segment (start 63.7282 38.9243) (end 63.7282 23.7982) (width 0.2) (layer "B.Cu") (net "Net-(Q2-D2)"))
 (segment (start 60.7448 41.9077) (end 63.7282 38.9243) (width 0.2) (layer "B.Cu") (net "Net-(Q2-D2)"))
 (segment (start 46.45 34) (end 47.0517 34) (width 0.2) (layer "F.Cu") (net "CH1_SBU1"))
 (segment (start 44.0957 36.956) (end 47.0517 34) (width 0.2) (layer "F.Cu") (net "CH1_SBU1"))
 (segment (start 62.0483 35.0034) (end 62.45 34.6017) (width 0.2) (layer "F.Cu") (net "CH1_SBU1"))
 (segment (start 29.956 36.956) (end 44.0957 36.956) (width 0.2) (layer "F.Cu") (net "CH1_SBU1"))
 (segment (start 62.45 34) (end 62.45 34.6017) (width 0.2) (layer "F.Cu") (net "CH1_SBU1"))
 (segment (start 62.45 34.6017) (end 62.45 42) (width 0.2) (layer "F.Cu") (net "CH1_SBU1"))
 (segment (start 48.0551 35.0034) (end 62.0483 35.0034) (width 0.2) (layer "F.Cu") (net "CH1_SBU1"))
 (segment (start 28.27 35.27) (end 29.956 36.956) (width 0.2) (layer "F.Cu") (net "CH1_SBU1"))
 (segment (start 47.0517 34) (end 48.0551 35.0034) (width 0.2) (layer "F.Cu") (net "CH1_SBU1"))
 (segment (start 37.2492 42) (end 36.9483 42) (width 0.2) (layer "F.Cu") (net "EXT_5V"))
 (segment (start 45.55 50) (end 45.55 50.6017) (width 0.2) (layer "F.Cu") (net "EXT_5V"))
 (segment (start 43.7966 41.3983) (end 36.9583 41.3983) (width 0.2) (layer "F.Cu") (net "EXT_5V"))
 (segment (start 36.9583 41.3983) (end 36.9483 41.4083) (width 0.2) (layer "F.Cu") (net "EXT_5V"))
 (segment (start 44.9483 49.6991) (end 44.9483 50) (width 0.2) (layer "F.Cu") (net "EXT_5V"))
 (segment (start 45.55 50) (end 44.9483 50) (width 0.2) (layer "F.Cu") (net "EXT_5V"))
 (segment (start 45.55 50.6017) (end 60.3466 50.6017) (width 0.2) (layer "F.Cu") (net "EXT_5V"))
 (segment (start 45.1 42) (end 44.3983 42) (width 0.2) (layer "F.Cu") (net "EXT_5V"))
 (segment (start 61.55 50) (end 60.9483 50) (width 0.2) (layer "F.Cu") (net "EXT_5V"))
 (segment (start 36.9483 41.4083) (end 36.9483 42) (width 0.2) (layer "F.Cu") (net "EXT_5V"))
 (segment (start 44.3983 42) (end 43.7966 41.3983) (width 0.2) (layer "F.Cu") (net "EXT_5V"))
 (segment (start 36.889 41.329) (end 36.9583 41.3983) (width 0.2) (layer "F.Cu") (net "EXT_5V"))
 (segment (start 37.55 42) (end 37.2492 42) (width 0.2) (layer "F.Cu") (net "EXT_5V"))
 (segment (start 60.3466 50.6017) (end 60.9483 50) (width 0.2) (layer "F.Cu") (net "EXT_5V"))
 (segment (start 37.2492 42) (end 44.9483 49.6991) (width 0.2) (layer "F.Cu") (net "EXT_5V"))
 (via (at 36.889 41.329) (size 0.6) (drill 0.3) (layers "F.Cu" "B.Cu") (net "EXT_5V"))
 (segment (start 24.46 34) (end 23.19 32.73) (width 0.2) (layer "B.Cu") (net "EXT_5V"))
 (segment (start 30.81 35.27) (end 29.54 34) (width 0.2) (layer "B.Cu") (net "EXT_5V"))
 (segment (start 30.81 35.27) (end 30.83 35.27) (width 0.2) (layer "B.Cu") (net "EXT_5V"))
 (segment (start 29.54 34) (end 24.46 34) (width 0.2) (layer "B.Cu") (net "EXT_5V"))
 (segment (start 30.83 35.27) (end 36.889 41.329) (width 0.2) (layer "B.Cu") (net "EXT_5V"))
 (segment (start 60.071 33.1227) (end 60.9483 34) (width 0.2) (layer "F.Cu") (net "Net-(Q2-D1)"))
 (segment (start 61.55 34) (end 60.9483 34) (width 0.2) (layer "F.Cu") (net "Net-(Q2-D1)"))
 (segment (start 61.05 23.7982) (end 60.3444 23.7982) (width 0.2) (layer "F.Cu") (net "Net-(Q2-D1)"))
 (segment (start 59.05 33.1227) (end 60.071 33.1227) (width 0.2) (layer "F.Cu") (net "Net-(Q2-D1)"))
 (segment (start 61.05 24.6999) (end 61.05 23.7982) (width 0.2) (layer "F.Cu") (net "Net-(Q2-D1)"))
 (via (at 60.3444 23.7982) (size 0.6) (drill 0.3) (layers "F.Cu" "B.Cu") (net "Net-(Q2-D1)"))
 (via (at 59.05 33.1227) (size 0.6) (drill 0.3) (layers "F.Cu" "B.Cu") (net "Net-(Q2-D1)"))
 (segment (start 59.05 25.0926) (end 60.3444 23.7982) (width 0.2) (layer "B.Cu") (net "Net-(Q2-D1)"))
 (segment (start 59.05 33.1227) (end 59.05 25.0926) (width 0.2) (layer "B.Cu") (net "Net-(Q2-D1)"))
 (segment (start 46.45 50) (end 49.8886 50) (width 0.2) (layer "F.Cu") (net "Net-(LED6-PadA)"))
 (segment (start 54 27.05) (end 50.8282 27.05) (width 0.2) (layer "F.Cu") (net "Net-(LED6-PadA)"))
 (via (at 49.8886 50) (size 0.6) (drill 0.3) (layers "F.Cu" "B.Cu") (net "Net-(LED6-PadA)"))
 (via (at 50.8282 27.05) (size 0.6) (drill 0.3) (layers "F.Cu" "B.Cu") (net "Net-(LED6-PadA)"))
 (segment (start 50.8282 49.0604) (end 49.8886 50) (width 0.2) (layer "B.Cu") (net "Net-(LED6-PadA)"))
 (segment (start 50.8282 27.05) (end 50.8282 49.0604) (width 0.2) (layer "B.Cu") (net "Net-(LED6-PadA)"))
 (segment (start 46.6511 27.0131) (end 47.0548 26.6094) (width 0.2) (layer "F.Cu") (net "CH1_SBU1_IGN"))
 (segment (start 54.45 50) (end 54.45 49.3983) (width 0.2) (layer "F.Cu") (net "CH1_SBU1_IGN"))
 (segment (start 61.05 27.3001) (end 57.5908 27.3001) (width 0.2) (layer "F.Cu") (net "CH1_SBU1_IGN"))
 (segment (start 57.5908 27.3001) (end 56.4265 26.1358) (width 0.2) (layer "F.Cu") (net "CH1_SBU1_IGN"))
 (segment (start 46.8819 25.3983) (end 47.0548 25.5712) (width 0.2) (layer "F.Cu") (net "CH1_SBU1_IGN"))
 (segment (start 45.55 25.3983) (end 46.8819 25.3983) (width 0.2) (layer "F.Cu") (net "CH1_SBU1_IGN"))
 (segment (start 47.0548 25.5712) (end 47.0548 26.1358) (width 0.2) (layer "F.Cu") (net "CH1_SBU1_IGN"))
 (segment (start 24.46 34) (end 24.46 32.2004) (width 0.2) (layer "F.Cu") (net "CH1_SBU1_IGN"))
 (segment (start 47.0548 26.6094) (end 47.0548 26.1358) (width 0.2) (layer "F.Cu") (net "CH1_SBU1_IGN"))
 (segment (start 24.46 32.2004) (end 30.4237 26.2367) (width 0.2) (layer "F.Cu") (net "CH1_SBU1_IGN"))
 (segment (start 40.2398 27.0131) (end 46.6511 27.0131) (width 0.2) (layer "F.Cu") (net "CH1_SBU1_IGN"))
 (segment (start 54.5669 49.3983) (end 54.45 49.3983) (width 0.2) (layer "F.Cu") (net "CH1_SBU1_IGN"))
 (segment (start 25.73 35.27) (end 24.46 34) (width 0.2) (layer "F.Cu") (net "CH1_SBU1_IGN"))
 (segment (start 54.7895 49.1757) (end 54.5669 49.3983) (width 0.2) (layer "F.Cu") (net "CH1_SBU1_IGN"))
 (segment (start 39.4634 26.2367) (end 40.2398 27.0131) (width 0.2) (layer "F.Cu") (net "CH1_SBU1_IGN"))
 (segment (start 30.4237 26.2367) (end 39.4634 26.2367) (width 0.2) (layer "F.Cu") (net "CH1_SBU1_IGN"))
 (segment (start 45.55 26) (end 45.55 25.3983) (width 0.2) (layer "F.Cu") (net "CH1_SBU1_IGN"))
 (segment (start 56.4265 26.1358) (end 47.0548 26.1358) (width 0.2) (layer "F.Cu") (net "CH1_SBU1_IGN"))
 (via (at 57.5908 27.3001) (size 0.6) (drill 0.3) (layers "F.Cu" "B.Cu") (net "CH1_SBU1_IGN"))
 (via (at 54.7895 49.1757) (size 0.6) (drill 0.3) (layers "F.Cu" "B.Cu") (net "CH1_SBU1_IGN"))
 (segment (start 54.7895 49.1757) (end 54.7895 30.1014) (width 0.2) (layer "B.Cu") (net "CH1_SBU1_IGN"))
 (segment (start 54.7895 30.1014) (end 57.5908 27.3001) (width 0.2) (layer "B.Cu") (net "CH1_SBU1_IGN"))
 (segment (start 42.4074 31.4591) (end 44.9483 34) (width 0.2) (layer "F.Cu") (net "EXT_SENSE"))
 (segment (start 45.55 34) (end 44.9483 34) (width 0.2) (layer "F.Cu") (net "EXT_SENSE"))
 (segment (start 29.5409 31.4591) (end 42.4074 31.4591) (width 0.2) (layer "F.Cu") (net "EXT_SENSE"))
 (segment (start 28.27 32.73) (end 29.5409 31.4591) (width 0.2) (layer "F.Cu") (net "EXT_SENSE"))
 (segment (start 37.7517 27) (end 37.9567 27) (width 0.2) (layer "F.Cu") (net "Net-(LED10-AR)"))
 (segment (start 44.55 47.8152) (end 50.7635 47.8152) (width 0.2) (layer "F.Cu") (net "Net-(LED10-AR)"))
 (segment (start 50.7635 47.8152) (end 52.9483 50) (width 0.2) (layer "F.Cu") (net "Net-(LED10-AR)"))
 (segment (start 53.55 50) (end 52.9483 50) (width 0.2) (layer "F.Cu") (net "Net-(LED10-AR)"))
 (segment (start 37.05 27) (end 37.7517 27) (width 0.2) (layer "F.Cu") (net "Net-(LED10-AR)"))
 (via (at 44.55 47.8152) (size 0.6) (drill 0.3) (layers "F.Cu" "B.Cu") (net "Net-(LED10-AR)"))
 (via (at 37.9567 27) (size 0.6) (drill 0.3) (layers "F.Cu" "B.Cu") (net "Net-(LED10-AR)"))
 (segment (start 44.55 33.5933) (end 37.9567 27) (width 0.2) (layer "B.Cu") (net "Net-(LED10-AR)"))
 (segment (start 44.55 47.8152) (end 44.55 33.5933) (width 0.2) (layer "B.Cu") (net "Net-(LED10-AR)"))
 (segment (start 38.95 27) (end 39.6517 27) (width 0.2) (layer "F.Cu") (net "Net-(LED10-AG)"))
 (segment (start 46.65 27.7017) (end 40.3534 27.7017) (width 0.2) (layer "F.Cu") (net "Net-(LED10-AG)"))
 (segment (start 40.3534 27.7017) (end 39.6517 27) (width 0.2) (layer "F.Cu") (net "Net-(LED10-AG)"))
 (segment (start 53.55 34) (end 52.9483 34) (width 0.2) (layer "F.Cu") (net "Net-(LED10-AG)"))
 (segment (start 52.9483 34) (end 46.65 27.7017) (width 0.2) (layer "F.Cu") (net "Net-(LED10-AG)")))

